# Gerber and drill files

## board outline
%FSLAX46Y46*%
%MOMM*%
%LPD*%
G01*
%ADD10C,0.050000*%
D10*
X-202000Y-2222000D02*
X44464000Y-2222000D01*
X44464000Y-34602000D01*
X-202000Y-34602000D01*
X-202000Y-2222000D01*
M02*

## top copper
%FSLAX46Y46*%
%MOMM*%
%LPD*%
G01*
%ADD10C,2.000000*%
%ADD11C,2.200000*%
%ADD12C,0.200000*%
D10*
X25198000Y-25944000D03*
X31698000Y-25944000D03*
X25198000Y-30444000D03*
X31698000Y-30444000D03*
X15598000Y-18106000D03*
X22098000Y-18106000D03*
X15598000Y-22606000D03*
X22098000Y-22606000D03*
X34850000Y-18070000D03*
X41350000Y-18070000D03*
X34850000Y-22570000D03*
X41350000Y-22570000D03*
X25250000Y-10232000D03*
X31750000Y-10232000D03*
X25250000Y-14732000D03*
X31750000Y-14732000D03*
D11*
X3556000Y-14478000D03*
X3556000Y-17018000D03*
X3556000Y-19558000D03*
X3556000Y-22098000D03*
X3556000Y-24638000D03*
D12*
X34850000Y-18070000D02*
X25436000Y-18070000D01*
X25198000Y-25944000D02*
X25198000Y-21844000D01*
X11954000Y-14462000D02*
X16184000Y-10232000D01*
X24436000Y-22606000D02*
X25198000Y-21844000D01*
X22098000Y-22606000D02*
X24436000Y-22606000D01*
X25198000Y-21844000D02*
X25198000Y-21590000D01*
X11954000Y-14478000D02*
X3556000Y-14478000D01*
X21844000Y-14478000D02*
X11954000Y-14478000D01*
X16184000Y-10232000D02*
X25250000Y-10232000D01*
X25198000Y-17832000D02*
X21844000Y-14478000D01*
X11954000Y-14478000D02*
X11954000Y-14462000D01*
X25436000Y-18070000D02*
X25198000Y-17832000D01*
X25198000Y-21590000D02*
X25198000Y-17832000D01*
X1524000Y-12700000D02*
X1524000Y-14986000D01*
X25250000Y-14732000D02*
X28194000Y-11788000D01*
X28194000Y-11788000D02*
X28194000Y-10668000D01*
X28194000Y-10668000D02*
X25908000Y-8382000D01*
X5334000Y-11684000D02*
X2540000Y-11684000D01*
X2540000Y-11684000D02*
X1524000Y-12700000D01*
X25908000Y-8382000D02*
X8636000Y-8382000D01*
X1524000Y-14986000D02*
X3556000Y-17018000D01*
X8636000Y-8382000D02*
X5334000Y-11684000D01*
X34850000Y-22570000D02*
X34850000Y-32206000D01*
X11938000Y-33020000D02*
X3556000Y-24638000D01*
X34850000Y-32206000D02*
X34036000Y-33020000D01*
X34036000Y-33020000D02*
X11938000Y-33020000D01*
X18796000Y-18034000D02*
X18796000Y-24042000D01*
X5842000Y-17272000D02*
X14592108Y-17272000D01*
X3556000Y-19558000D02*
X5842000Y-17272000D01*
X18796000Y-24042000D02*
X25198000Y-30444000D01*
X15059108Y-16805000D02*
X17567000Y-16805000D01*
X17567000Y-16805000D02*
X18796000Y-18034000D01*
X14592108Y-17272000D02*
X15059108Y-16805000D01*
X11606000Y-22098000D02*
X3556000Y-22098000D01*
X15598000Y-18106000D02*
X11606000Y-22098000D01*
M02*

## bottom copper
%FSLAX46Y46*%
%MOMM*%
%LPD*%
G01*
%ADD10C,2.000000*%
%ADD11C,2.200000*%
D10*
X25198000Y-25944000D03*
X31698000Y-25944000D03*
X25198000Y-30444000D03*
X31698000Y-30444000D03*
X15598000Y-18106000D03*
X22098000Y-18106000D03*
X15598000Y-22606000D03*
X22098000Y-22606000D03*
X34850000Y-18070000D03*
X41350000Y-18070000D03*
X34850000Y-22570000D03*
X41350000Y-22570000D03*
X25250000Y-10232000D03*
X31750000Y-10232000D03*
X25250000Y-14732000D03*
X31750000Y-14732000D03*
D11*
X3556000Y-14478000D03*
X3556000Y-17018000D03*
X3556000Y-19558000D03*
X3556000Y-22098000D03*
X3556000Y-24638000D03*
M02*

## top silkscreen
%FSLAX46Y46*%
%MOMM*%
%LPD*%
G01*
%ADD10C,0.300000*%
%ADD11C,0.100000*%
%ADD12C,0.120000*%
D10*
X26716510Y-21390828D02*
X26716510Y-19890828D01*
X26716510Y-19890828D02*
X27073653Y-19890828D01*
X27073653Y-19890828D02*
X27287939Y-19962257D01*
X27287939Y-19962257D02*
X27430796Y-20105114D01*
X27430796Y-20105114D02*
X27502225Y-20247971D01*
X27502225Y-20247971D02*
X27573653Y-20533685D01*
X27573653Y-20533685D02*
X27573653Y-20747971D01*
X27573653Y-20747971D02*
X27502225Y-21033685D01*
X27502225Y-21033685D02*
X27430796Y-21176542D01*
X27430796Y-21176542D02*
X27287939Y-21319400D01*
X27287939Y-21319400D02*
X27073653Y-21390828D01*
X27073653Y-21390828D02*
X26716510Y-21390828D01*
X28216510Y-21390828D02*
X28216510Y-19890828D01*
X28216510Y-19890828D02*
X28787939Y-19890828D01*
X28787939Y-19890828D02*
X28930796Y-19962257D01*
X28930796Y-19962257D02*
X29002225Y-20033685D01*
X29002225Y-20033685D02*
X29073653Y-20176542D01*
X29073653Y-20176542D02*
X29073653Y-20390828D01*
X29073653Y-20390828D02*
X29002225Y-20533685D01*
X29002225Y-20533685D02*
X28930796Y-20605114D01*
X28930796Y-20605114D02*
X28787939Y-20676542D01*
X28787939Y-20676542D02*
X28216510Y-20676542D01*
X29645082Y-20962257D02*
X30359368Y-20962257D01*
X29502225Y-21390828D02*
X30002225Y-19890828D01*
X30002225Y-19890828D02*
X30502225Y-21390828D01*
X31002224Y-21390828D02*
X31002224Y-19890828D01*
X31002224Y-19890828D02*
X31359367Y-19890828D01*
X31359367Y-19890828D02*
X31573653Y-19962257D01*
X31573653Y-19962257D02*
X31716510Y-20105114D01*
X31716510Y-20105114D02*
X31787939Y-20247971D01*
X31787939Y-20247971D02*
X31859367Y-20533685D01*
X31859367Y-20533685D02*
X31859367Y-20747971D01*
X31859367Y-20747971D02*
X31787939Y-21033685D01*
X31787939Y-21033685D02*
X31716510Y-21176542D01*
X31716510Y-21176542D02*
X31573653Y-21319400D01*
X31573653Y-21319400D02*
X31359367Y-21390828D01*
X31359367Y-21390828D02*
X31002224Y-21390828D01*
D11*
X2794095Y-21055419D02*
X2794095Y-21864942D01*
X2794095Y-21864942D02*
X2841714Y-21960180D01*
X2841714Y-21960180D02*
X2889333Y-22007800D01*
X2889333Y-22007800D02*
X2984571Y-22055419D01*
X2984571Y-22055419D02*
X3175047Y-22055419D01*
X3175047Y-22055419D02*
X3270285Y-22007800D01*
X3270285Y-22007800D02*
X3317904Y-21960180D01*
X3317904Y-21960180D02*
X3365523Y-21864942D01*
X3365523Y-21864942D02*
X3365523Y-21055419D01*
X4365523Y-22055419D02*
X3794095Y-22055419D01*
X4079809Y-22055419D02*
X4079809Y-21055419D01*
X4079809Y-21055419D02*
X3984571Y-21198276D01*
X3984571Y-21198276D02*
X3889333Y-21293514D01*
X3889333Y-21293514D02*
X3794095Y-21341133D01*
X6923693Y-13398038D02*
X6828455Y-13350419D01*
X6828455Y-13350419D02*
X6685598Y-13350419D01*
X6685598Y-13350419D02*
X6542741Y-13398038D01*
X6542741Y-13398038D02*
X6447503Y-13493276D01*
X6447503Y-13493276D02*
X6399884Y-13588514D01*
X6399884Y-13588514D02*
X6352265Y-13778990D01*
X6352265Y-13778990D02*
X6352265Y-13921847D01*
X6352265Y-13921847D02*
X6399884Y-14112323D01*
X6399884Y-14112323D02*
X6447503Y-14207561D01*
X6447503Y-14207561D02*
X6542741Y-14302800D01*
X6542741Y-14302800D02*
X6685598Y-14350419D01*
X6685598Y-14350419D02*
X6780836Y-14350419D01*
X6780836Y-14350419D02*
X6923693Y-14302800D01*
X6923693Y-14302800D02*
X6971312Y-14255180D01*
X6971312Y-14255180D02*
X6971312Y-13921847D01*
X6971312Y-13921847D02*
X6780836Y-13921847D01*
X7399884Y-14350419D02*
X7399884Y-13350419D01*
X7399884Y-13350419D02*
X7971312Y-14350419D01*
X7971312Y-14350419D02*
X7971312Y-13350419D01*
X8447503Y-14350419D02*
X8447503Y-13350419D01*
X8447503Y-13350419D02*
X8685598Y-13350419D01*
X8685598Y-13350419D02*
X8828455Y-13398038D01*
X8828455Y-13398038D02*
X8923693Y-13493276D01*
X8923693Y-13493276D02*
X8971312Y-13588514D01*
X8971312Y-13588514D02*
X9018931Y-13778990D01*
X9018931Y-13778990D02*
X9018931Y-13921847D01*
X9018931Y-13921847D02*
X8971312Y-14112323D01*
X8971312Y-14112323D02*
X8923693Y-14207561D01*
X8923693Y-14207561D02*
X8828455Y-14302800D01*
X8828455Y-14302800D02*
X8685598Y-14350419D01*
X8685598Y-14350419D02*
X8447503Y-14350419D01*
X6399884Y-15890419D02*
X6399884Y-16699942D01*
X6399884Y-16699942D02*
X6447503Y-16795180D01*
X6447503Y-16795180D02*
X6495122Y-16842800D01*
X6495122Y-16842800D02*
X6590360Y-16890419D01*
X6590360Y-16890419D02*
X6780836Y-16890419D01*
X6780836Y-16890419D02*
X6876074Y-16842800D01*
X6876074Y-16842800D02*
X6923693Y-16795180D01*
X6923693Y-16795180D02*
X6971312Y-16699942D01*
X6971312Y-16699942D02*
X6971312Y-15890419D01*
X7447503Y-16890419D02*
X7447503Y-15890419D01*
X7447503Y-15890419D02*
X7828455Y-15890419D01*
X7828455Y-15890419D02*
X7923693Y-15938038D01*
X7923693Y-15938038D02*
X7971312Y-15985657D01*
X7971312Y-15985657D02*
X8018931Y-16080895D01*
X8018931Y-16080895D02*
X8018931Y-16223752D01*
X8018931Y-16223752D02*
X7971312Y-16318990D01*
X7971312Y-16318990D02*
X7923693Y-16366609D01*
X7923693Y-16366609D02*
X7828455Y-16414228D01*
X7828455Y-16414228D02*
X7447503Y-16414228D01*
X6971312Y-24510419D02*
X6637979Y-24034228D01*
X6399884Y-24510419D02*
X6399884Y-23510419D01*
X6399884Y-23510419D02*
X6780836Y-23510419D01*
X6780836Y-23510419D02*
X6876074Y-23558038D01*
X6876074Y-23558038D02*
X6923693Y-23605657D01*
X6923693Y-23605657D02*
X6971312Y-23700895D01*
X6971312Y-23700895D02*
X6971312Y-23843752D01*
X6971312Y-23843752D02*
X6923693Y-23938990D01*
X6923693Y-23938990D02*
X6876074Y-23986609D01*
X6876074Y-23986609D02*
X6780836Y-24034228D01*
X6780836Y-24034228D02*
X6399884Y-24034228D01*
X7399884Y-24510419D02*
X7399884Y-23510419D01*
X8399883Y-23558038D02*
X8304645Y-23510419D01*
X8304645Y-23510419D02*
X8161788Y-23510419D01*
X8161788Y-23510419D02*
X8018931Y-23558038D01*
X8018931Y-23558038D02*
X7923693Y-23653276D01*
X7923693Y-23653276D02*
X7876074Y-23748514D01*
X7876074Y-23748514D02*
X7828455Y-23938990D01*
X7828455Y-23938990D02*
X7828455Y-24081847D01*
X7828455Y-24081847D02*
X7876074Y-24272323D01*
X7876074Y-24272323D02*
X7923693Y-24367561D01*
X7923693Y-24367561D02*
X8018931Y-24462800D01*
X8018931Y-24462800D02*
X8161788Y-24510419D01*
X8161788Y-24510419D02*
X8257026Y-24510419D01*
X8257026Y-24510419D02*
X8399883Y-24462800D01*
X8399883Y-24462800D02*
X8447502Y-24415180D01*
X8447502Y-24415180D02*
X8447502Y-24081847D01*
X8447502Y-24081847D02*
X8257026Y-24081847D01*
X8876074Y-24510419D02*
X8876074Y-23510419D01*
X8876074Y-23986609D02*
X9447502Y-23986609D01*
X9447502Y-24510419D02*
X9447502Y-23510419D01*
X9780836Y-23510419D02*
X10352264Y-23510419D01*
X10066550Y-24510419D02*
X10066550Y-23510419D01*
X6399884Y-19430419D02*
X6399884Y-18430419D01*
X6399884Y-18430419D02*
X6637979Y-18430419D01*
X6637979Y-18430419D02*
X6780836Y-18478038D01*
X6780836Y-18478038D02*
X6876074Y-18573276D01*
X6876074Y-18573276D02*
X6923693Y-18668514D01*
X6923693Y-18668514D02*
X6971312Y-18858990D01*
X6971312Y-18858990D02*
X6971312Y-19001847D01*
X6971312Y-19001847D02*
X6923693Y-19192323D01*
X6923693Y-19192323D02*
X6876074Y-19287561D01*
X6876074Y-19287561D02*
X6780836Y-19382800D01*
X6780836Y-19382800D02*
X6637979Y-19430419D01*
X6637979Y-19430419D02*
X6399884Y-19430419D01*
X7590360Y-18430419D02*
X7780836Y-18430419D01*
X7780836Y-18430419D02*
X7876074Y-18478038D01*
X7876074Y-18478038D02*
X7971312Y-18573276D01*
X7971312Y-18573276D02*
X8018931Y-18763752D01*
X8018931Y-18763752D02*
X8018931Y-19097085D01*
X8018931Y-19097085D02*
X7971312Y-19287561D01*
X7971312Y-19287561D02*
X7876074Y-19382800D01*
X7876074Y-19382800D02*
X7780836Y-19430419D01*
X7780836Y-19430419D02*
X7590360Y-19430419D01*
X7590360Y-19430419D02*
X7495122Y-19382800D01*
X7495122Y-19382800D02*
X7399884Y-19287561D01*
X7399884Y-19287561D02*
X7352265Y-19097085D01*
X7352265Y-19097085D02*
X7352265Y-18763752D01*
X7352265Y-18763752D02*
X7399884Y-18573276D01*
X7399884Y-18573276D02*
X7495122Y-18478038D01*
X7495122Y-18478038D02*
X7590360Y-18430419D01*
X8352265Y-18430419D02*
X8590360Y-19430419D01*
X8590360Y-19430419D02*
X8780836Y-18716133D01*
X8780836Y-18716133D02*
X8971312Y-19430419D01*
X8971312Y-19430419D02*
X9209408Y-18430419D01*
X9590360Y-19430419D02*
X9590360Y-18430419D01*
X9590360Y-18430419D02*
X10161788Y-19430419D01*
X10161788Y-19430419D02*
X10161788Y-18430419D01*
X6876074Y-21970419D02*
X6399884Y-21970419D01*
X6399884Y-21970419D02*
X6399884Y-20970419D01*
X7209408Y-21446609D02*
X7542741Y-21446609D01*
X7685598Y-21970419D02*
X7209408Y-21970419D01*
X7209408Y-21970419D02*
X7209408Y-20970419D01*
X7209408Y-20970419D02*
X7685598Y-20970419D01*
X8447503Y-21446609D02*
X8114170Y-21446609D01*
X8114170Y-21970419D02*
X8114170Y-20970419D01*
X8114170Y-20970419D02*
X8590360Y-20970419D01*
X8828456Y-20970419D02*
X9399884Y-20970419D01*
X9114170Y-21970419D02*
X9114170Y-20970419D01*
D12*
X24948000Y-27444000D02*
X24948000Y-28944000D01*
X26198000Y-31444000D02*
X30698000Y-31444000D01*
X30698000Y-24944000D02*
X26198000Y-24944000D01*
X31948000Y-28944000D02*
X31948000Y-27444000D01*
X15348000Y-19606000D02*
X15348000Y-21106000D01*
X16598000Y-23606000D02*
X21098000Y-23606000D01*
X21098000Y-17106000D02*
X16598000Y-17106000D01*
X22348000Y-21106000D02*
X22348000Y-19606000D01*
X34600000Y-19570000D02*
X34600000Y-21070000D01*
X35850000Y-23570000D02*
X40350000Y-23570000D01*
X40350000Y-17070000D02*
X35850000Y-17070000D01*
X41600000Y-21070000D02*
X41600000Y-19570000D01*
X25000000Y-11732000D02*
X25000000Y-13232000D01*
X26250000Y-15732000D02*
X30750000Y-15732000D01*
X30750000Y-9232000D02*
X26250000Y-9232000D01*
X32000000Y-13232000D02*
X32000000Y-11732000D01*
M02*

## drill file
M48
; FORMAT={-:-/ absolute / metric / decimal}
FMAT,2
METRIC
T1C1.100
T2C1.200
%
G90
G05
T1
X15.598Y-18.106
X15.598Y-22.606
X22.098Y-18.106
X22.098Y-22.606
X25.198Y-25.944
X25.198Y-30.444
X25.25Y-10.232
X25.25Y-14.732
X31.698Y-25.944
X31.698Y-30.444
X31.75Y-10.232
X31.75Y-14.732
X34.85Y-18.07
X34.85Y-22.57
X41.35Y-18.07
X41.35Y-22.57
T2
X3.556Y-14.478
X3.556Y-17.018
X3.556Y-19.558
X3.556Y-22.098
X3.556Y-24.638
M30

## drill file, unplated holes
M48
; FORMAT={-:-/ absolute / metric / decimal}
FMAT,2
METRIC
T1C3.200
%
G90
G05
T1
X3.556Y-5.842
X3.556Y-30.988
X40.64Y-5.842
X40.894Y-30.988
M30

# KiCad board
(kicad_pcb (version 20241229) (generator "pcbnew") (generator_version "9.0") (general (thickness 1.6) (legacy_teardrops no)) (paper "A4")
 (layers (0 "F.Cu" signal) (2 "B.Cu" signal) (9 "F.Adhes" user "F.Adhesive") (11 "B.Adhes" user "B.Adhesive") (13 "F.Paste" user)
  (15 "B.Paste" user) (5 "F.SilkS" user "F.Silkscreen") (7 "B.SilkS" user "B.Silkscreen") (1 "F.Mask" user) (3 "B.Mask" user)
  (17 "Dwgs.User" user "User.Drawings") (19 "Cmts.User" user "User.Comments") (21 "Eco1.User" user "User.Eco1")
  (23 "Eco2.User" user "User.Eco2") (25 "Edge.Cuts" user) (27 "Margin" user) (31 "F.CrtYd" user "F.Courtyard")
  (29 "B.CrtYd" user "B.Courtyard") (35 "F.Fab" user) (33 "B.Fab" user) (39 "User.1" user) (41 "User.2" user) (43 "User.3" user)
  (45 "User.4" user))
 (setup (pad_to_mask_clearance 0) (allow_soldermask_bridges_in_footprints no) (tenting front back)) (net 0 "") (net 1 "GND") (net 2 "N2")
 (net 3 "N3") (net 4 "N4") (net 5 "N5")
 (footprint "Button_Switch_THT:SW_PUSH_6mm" (layer "F.Cu") (at 25.198 25.944)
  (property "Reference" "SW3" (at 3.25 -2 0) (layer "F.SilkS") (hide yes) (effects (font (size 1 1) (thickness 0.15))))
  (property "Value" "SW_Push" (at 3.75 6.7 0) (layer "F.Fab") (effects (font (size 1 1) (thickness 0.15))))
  (fp_line (start -0.25 1.5) (end -0.25 3) (stroke (width 0.12) (type solid)) (layer "F.SilkS"))
  (fp_line (start 1 5.5) (end 5.5 5.5) (stroke (width 0.12) (type solid)) (layer "F.SilkS"))
  (fp_line (start 5.5 -1) (end 1 -1) (stroke (width 0.12) (type solid)) (layer "F.SilkS"))
  (fp_line (start 6.75 3) (end 6.75 1.5) (stroke (width 0.12) (type solid)) (layer "F.SilkS"))
  (pad "1" thru_hole circle (at 0 0 90) (size 2 2) (drill 1.1) (layers "*.Cu" "*.Mask") (remove_unused_layers no) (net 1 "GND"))
  (pad "1" thru_hole circle (at 6.5 0 90) (size 2 2) (drill 1.1) (layers "*.Cu" "*.Mask") (remove_unused_layers no) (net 1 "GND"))
  (pad "2" thru_hole circle (at 0 4.5 90) (size 2 2) (drill 1.1) (layers "*.Cu" "*.Mask") (remove_unused_layers no) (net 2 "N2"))
  (pad "2" thru_hole circle (at 6.5 4.5 90) (size 2 2) (drill 1.1) (layers "*.Cu" "*.Mask") (remove_unused_layers no) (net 2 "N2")))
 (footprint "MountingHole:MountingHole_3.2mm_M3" (layer "F.Cu") (at 3.556 30.988)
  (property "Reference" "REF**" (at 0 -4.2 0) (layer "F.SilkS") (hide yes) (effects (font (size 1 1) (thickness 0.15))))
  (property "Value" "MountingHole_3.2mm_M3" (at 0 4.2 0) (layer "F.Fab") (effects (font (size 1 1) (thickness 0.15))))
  (pad "" np_thru_hole circle (at 0 0) (size 3.2 3.2) (drill 3.2) (layers "*.Cu" "*.Mask")))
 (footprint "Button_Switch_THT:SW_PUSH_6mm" (layer "F.Cu") (at 15.598 18.106)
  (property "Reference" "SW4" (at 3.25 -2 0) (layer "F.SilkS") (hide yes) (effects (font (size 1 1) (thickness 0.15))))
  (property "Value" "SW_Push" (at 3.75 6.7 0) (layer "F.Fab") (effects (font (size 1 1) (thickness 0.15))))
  (fp_line (start -0.25 1.5) (end -0.25 3) (stroke (width 0.12) (type solid)) (layer "F.SilkS"))
  (fp_line (start 1 5.5) (end 5.5 5.5) (stroke (width 0.12) (type solid)) (layer "F.SilkS"))
  (fp_line (start 5.5 -1) (end 1 -1) (stroke (width 0.12) (type solid)) (layer "F.SilkS"))
  (fp_line (start 6.75 3) (end 6.75 1.5) (stroke (width 0.12) (type solid)) (layer "F.SilkS"))
  (pad "1" thru_hole circle (at 0 0 90) (size 2 2) (drill 1.1) (layers "*.Cu" "*.Mask") (remove_unused_layers no) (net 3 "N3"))
  (pad "1" thru_hole circle (at 6.5 0 90) (size 2 2) (drill 1.1) (layers "*.Cu" "*.Mask") (remove_unused_layers no) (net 3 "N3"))
  (pad "2" thru_hole circle (at 0 4.5 90) (size 2 2) (drill 1.1) (layers "*.Cu" "*.Mask") (remove_unused_layers no) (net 1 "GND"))
  (pad "2" thru_hole circle (at 6.5 4.5 90) (size 2 2) (drill 1.1) (layers "*.Cu" "*.Mask") (remove_unused_layers no) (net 1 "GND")))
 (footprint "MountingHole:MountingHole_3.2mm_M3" (layer "F.Cu") (at 3.556 5.842)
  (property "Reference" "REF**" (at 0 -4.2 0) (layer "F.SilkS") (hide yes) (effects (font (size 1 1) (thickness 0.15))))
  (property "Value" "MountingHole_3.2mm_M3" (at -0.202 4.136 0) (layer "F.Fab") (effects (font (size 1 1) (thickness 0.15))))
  (pad "" np_thru_hole circle (at 0 0) (size 3.2 3.2) (drill 3.2) (layers "*.Cu" "*.Mask")))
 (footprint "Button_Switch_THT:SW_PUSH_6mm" (layer "F.Cu") (at 34.85 18.07)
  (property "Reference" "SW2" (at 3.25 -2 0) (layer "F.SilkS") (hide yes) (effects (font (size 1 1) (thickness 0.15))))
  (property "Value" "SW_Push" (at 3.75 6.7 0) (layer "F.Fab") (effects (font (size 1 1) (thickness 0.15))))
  (fp_line (start -0.25 1.5) (end -0.25 3) (stroke (width 0.12) (type solid)) (layer "F.SilkS"))
  (fp_line (start 1 5.5) (end 5.5 5.5) (stroke (width 0.12) (type solid)) (layer "F.SilkS"))
  (fp_line (start 5.5 -1) (end 1 -1) (stroke (width 0.12) (type solid)) (layer "F.SilkS"))
  (fp_line (start 6.75 3) (end 6.75 1.5) (stroke (width 0.12) (type solid)) (layer "F.SilkS"))
  (pad "1" thru_hole circle (at 0 0 90) (size 2 2) (drill 1.1) (layers "*.Cu" "*.Mask") (remove_unused_layers no) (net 1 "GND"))
  (pad "1" thru_hole circle (at 6.5 0 90) (size 2 2) (drill 1.1) (layers "*.Cu" "*.Mask") (remove_unused_layers no) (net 1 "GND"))
  (pad "2" thru_hole circle (at 0 4.5 90) (size 2 2) (drill 1.1) (layers "*.Cu" "*.Mask") (remove_unused_layers no) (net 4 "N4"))
  (pad "2" thru_hole circle (at 6.5 4.5 90) (size 2 2) (drill 1.1) (layers "*.Cu" "*.Mask") (remove_unused_layers no) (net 4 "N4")))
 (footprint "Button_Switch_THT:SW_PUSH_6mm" (layer "F.Cu") (at 25.25 10.232)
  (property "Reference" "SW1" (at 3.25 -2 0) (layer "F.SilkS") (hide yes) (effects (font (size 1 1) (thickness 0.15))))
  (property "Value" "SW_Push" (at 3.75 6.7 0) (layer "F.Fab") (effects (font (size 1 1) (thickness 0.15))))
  (fp_line (start -0.25 1.5) (end -0.25 3) (stroke (width 0.12) (type solid)) (layer "F.SilkS"))
  (fp_line (start 1 5.5) (end 5.5 5.5) (stroke (width 0.12) (type solid)) (layer "F.SilkS"))
  (fp_line (start 5.5 -1) (end 1 -1) (stroke (width 0.12) (type solid)) (layer "F.SilkS"))
  (fp_line (start 6.75 3) (end 6.75 1.5) (stroke (width 0.12) (type solid)) (layer "F.SilkS"))
  (pad "1" thru_hole circle (at 0 0 90) (size 2 2) (drill 1.1) (layers "*.Cu" "*.Mask") (remove_unused_layers no) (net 1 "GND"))
  (pad "1" thru_hole circle (at 6.5 0 90) (size 2 2) (drill 1.1) (layers "*.Cu" "*.Mask") (remove_unused_layers no) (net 1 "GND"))
  (pad "2" thru_hole circle (at 0 4.5 90) (size 2 2) (drill 1.1) (layers "*.Cu" "*.Mask") (remove_unused_layers no) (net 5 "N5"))
  (pad "2" thru_hole circle (at 6.5 4.5 90) (size 2 2) (drill 1.1) (layers "*.Cu" "*.Mask") (remove_unused_layers no) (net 5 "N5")))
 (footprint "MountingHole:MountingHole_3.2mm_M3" (layer "F.Cu") (at 40.64 5.842)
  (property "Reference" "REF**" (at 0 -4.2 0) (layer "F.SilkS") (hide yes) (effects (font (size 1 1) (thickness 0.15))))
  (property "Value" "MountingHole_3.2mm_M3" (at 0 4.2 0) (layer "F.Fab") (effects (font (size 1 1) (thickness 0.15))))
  (pad "" np_thru_hole circle (at 0 0) (size 3.2 3.2) (drill 3.2) (layers "*.Cu" "*.Mask")))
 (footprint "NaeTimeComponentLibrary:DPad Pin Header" (layer "F.Cu") (at 3.556 19.558)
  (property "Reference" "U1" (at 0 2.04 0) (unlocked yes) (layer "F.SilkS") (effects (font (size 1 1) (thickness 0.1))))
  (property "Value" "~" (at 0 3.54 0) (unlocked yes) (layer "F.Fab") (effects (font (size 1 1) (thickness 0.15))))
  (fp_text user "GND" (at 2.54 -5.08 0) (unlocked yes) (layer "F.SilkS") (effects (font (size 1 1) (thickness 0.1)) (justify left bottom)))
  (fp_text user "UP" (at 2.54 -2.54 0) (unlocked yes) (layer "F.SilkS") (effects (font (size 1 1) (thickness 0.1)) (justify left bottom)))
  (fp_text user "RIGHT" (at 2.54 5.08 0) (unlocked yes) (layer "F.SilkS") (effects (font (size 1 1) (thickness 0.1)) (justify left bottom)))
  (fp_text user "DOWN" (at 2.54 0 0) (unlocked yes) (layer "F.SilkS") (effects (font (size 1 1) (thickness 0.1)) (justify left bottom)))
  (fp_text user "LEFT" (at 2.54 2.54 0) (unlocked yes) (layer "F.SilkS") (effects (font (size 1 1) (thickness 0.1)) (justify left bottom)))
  (pad "1" thru_hole circle (at 0 -5.08) (size 2.2 2.2) (drill 1.2) (layers "*.Cu" "*.Mask") (remove_unused_layers no) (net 1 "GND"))
  (pad "2" thru_hole circle (at 0 -2.54) (size 2.2 2.2) (drill 1.2) (layers "*.Cu" "*.Mask") (remove_unused_layers no) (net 5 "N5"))
  (pad "3" thru_hole circle (at 0 0) (size 2.2 2.2) (drill 1.2) (layers "*.Cu" "*.Mask") (remove_unused_layers no) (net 2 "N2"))
  (pad "4" thru_hole circle (at 0 2.54) (size 2.2 2.2) (drill 1.2) (layers "*.Cu" "*.Mask") (remove_unused_layers no) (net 3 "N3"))
  (pad "5" thru_hole circle (at 0 5.08) (size 2.2 2.2) (drill 1.2) (layers "*.Cu" "*.Mask") (remove_unused_layers no) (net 4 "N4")))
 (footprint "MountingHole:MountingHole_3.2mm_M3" (layer "F.Cu") (at 40.894 30.988)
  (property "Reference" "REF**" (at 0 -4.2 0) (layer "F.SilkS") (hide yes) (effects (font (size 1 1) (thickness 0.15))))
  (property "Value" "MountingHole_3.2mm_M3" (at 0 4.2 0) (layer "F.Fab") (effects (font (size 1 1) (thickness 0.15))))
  (pad "" np_thru_hole circle (at 0 0) (size 3.2 3.2) (drill 3.2) (layers "*.Cu" "*.Mask")))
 (gr_rect (start -0.202 2.222) (end 44.464 34.602) (stroke (width 0.05) (type solid)) (fill no) (layer "Edge.Cuts"))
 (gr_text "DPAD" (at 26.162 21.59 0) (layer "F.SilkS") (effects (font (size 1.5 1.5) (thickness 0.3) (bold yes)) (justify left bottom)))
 (segment (start 34.85 18.07) (end 25.436 18.07) (width 0.2) (layer "F.Cu") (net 1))
 (segment (start 25.198 25.944) (end 25.198 21.844) (width 0.2) (layer "F.Cu") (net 1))
 (segment (start 11.954 14.462) (end 16.184 10.232) (width 0.2) (layer "F.Cu") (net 1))
 (segment (start 24.436 22.606) (end 25.198 21.844) (width 0.2) (layer "F.Cu") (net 1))
 (segment (start 22.098 22.606) (end 24.436 22.606) (width 0.2) (layer "F.Cu") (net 1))
 (segment (start 25.198 21.844) (end 25.198 21.59) (width 0.2) (layer "F.Cu") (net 1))
 (segment (start 11.954 14.478) (end 3.556 14.478) (width 0.2) (layer "F.Cu") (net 1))
 (segment (start 21.844 14.478) (end 11.954 14.478) (width 0.2) (layer "F.Cu") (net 1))
 (segment (start 16.184 10.232) (end 25.25 10.232) (width 0.2) (layer "F.Cu") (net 1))
 (segment (start 25.198 17.832) (end 21.844 14.478) (width 0.2) (layer "F.Cu") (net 1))
 (segment (start 11.954 14.478) (end 11.954 14.462) (width 0.2) (layer "F.Cu") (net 1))
 (segment (start 25.436 18.07) (end 25.198 17.832) (width 0.2) (layer "F.Cu") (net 1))
 (segment (start 25.198 21.59) (end 25.198 17.832) (width 0.2) (layer "F.Cu") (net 1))
 (segment (start 1.524 12.7) (end 1.524 14.986) (width 0.2) (layer "F.Cu") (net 5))
 (segment (start 25.25 14.732) (end 28.194 11.788) (width 0.2) (layer "F.Cu") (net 5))
 (segment (start 28.194 11.788) (end 28.194 10.668) (width 0.2) (layer "F.Cu") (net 5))
 (segment (start 28.194 10.668) (end 25.908 8.382) (width 0.2) (layer "F.Cu") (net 5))
 (segment (start 5.334 11.684) (end 2.54 11.684) (width 0.2) (layer "F.Cu") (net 5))
 (segment (start 2.54 11.684) (end 1.524 12.7) (width 0.2) (layer "F.Cu") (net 5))
 (segment (start 25.908 8.382) (end 8.636 8.382) (width 0.2) (layer "F.Cu") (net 5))
 (segment (start 1.524 14.986) (end 3.556 17.018) (width 0.2) (layer "F.Cu") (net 5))
 (segment (start 8.636 8.382) (end 5.334 11.684) (width 0.2) (layer "F.Cu") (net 5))
 (segment (start 34.85 22.57) (end 34.85 32.206) (width 0.2) (layer "F.Cu") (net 4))
 (segment (start 11.938 33.02) (end 3.556 24.638) (width 0.2) (layer "F.Cu") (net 4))
 (segment (start 34.85 32.206) (end 34.036 33.02) (width 0.2) (layer "F.Cu") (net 4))
 (segment (start 34.036 33.02) (end 11.938 33.02) (width 0.2) (layer "F.Cu") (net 4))
 (segment (start 18.796 18.034) (end 18.796 24.042) (width 0.2) (layer "F.Cu") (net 2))
 (segment (start 5.842 17.272) (end 14.592108 17.272) (width 0.2) (layer "F.Cu") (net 2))
 (segment (start 3.556 19.558) (end 5.842 17.272) (width 0.2) (layer "F.Cu") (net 2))
 (segment (start 18.796 24.042) (end 25.198 30.444) (width 0.2) (layer "F.Cu") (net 2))
 (segment (start 15.059108 16.805) (end 17.567 16.805) (width 0.2) (layer "F.Cu") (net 2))
 (segment (start 17.567 16.805) (end 18.796 18.034) (width 0.2) (layer "F.Cu") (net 2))
 (segment (start 14.592108 17.272) (end 15.059108 16.805) (width 0.2) (layer "F.Cu") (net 2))
 (segment (start 11.606 22.098) (end 3.556 22.098) (width 0.2) (layer "F.Cu") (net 3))
 (segment (start 15.598 18.106) (end 11.606 22.098) (width 0.2) (layer "F.Cu") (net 3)))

